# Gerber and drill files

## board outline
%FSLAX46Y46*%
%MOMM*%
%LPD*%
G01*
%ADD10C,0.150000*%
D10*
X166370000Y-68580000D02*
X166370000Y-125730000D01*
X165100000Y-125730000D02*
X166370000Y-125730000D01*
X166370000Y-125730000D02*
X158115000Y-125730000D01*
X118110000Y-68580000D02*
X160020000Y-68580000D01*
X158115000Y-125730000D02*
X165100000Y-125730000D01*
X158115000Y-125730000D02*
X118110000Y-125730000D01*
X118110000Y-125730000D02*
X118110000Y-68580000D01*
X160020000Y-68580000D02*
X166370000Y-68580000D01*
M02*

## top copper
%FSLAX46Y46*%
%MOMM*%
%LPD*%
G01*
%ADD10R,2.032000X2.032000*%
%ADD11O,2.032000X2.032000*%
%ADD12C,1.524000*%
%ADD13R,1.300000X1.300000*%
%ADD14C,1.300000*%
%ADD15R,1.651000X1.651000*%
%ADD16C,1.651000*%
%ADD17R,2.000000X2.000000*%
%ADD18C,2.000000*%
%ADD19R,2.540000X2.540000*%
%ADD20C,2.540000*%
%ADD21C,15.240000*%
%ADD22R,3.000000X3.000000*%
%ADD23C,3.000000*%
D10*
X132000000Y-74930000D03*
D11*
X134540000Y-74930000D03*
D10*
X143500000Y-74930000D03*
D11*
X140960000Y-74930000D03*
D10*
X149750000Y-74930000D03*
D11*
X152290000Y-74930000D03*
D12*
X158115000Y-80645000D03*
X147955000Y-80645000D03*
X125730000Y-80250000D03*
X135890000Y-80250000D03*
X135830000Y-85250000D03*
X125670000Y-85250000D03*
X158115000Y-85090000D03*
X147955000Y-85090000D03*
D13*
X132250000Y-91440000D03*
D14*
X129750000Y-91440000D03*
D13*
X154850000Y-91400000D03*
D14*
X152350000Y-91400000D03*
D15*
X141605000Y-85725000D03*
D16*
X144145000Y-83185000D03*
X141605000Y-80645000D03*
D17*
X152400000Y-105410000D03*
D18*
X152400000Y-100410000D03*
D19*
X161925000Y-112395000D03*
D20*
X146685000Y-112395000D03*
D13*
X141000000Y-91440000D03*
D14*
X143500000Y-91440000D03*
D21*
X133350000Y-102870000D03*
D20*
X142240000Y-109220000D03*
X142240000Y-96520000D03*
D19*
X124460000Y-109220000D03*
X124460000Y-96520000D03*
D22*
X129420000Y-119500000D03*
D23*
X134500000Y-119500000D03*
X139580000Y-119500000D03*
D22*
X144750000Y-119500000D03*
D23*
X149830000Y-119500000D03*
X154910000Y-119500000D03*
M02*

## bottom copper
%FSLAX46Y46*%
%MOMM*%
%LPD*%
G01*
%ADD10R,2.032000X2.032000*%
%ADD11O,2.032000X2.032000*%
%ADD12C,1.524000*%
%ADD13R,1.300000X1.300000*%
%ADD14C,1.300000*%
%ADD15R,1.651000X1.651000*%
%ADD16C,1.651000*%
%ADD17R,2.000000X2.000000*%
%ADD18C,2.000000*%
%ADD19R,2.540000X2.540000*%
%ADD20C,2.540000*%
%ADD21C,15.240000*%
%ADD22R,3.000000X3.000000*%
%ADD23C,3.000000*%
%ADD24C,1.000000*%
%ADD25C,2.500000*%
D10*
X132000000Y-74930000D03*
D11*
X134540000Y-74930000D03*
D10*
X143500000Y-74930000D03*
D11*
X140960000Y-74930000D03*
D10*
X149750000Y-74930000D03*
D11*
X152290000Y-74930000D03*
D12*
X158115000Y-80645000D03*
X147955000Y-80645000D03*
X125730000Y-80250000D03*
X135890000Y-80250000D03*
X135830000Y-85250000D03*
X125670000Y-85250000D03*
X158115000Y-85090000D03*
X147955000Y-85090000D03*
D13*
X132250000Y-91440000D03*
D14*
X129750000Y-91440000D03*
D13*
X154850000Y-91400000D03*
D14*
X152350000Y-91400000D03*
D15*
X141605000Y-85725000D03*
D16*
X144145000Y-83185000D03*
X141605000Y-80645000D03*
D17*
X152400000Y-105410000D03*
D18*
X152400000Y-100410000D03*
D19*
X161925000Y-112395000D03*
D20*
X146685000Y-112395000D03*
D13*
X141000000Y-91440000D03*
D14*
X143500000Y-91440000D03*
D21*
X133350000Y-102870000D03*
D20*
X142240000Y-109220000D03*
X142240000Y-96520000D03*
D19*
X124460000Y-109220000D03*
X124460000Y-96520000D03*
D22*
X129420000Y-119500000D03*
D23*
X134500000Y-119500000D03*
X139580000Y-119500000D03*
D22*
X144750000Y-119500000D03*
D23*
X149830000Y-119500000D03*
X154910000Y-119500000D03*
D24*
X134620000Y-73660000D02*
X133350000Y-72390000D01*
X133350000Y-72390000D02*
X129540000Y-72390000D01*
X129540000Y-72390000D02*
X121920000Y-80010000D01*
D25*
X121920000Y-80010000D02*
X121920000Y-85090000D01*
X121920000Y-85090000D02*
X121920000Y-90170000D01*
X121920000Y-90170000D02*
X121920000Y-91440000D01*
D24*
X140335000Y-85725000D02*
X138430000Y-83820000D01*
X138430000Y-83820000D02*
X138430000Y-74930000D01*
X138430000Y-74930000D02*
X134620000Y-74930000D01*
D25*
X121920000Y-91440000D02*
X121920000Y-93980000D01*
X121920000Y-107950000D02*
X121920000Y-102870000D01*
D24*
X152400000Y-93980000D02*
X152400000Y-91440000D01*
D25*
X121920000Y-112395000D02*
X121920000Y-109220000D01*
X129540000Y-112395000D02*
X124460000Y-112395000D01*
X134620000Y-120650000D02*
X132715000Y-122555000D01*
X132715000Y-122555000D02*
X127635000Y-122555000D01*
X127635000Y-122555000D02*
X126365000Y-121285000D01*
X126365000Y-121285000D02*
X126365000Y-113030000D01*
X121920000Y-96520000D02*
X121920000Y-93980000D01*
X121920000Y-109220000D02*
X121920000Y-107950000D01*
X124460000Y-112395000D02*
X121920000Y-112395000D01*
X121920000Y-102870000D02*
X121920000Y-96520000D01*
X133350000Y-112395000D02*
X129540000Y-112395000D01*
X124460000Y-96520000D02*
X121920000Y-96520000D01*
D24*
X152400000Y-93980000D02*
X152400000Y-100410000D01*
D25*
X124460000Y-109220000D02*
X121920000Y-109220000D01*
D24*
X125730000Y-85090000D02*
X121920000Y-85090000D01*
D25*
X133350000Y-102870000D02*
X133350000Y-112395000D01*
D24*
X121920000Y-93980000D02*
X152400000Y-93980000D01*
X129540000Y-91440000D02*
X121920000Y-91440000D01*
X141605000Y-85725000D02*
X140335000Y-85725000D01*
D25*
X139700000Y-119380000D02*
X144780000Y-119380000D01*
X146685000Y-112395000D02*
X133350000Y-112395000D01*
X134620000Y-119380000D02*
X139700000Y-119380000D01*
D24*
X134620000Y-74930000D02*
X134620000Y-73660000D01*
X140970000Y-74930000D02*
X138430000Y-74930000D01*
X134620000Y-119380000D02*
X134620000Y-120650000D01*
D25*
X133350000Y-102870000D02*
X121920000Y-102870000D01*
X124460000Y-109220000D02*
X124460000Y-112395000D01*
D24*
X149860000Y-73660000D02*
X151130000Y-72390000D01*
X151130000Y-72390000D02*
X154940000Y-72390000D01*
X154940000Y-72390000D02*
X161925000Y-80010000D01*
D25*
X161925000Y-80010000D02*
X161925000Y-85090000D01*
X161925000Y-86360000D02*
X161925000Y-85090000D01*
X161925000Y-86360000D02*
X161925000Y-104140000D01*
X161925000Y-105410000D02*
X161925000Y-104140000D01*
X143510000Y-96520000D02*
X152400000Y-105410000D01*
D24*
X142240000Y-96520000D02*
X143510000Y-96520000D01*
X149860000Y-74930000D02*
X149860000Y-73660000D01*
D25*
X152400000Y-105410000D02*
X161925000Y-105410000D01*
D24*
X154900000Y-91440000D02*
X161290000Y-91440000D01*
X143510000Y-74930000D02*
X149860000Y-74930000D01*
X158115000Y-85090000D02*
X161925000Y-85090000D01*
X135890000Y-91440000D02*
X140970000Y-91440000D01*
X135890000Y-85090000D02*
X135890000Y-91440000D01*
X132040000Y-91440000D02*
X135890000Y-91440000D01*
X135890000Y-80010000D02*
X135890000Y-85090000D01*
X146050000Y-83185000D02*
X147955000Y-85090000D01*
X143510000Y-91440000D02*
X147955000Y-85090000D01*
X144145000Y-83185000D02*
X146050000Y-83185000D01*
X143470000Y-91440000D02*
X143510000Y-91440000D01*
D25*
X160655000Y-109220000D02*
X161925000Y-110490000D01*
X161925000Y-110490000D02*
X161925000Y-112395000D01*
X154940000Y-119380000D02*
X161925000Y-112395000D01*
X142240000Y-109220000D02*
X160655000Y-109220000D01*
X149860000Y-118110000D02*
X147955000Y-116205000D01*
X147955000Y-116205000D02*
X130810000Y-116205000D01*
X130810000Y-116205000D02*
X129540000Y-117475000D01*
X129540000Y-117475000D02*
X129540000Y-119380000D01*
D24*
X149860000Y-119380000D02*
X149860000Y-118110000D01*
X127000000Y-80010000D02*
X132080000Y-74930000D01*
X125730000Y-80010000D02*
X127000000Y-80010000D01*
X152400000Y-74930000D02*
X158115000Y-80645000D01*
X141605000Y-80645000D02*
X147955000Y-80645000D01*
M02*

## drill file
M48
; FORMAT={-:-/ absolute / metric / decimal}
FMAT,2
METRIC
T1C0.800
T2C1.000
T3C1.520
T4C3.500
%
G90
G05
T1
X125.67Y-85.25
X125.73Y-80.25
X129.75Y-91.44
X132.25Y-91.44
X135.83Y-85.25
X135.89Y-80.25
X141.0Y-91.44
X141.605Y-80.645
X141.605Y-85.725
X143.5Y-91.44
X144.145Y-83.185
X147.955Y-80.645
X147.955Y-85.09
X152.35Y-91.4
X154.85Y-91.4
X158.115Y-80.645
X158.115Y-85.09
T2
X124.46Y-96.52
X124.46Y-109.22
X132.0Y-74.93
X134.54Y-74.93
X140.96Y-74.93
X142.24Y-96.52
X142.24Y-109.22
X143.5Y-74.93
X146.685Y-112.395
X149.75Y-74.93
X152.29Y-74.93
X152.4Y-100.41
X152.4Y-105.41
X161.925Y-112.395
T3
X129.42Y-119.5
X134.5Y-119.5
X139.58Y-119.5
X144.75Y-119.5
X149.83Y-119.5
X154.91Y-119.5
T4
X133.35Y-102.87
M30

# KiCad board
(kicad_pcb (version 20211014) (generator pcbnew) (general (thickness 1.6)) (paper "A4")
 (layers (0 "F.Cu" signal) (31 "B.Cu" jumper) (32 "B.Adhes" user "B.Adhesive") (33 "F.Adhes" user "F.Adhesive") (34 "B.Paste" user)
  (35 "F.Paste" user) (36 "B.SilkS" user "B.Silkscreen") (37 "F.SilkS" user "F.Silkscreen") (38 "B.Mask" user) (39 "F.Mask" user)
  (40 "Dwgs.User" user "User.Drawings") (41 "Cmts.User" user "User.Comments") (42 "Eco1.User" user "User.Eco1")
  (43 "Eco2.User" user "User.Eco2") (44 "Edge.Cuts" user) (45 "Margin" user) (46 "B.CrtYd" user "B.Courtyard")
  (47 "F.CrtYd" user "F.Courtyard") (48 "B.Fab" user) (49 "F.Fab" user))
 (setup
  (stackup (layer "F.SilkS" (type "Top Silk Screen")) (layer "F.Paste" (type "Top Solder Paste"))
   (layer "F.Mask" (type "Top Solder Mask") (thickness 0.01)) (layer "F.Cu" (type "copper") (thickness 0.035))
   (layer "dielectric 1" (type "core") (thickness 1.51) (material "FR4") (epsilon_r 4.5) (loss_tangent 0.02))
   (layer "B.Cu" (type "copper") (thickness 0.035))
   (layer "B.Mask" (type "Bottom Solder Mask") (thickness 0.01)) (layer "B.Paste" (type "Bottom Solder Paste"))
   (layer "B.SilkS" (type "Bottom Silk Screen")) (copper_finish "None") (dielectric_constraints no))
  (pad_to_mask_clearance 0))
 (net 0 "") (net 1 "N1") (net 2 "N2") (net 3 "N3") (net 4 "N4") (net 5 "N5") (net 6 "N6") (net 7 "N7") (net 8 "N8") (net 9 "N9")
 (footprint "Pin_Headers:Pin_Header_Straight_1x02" (layer "F.Cu") (at 132 74.93 90)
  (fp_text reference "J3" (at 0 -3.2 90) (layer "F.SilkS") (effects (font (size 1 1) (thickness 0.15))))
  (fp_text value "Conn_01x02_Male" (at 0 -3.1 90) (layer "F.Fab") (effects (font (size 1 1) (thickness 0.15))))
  (pad "1" thru_hole rect locked (at 0 0 90) (size 2.032 2.032) (drill 1) (layers *.Cu *.Mask) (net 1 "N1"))
  (pad "2" thru_hole oval locked (at 0 2.54 90) (size 2.032 2.032) (drill 1) (layers *.Cu *.Mask) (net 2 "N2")))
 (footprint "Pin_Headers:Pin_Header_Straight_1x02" (layer "F.Cu") (at 143.5 74.93 -90)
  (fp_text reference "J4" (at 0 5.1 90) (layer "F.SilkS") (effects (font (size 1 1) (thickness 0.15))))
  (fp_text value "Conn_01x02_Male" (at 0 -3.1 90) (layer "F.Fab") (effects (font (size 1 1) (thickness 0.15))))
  (pad "1" thru_hole rect locked (at 0 0 270) (size 2.032 2.032) (drill 1) (layers *.Cu *.Mask) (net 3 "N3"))
  (pad "2" thru_hole oval locked (at 0 2.54 270) (size 2.032 2.032) (drill 1) (layers *.Cu *.Mask) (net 2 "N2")))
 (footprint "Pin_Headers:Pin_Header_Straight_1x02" (layer "F.Cu") (at 149.75 74.93 90)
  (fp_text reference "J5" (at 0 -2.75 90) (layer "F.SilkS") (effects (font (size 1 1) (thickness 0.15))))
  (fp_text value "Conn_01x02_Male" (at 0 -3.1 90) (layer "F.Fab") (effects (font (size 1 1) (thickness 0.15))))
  (pad "1" thru_hole rect locked (at 0 0 90) (size 2.032 2.032) (drill 1) (layers *.Cu *.Mask) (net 3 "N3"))
  (pad "2" thru_hole oval locked (at 0 2.54 90) (size 2.032 2.032) (drill 1) (layers *.Cu *.Mask) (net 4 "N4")))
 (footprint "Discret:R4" (layer "F.Cu") (at 153.035 80.645 180)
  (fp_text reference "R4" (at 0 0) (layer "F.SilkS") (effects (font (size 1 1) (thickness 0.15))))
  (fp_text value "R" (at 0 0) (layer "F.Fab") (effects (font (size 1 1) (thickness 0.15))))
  (pad "1" thru_hole circle locked (at -5.08 0 180) (size 1.524 1.524) (drill 0.8) (layers *.Cu *.Mask) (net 4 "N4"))
  (pad "2" thru_hole circle locked (at 5.08 0 180) (size 1.524 1.524) (drill 0.8) (layers *.Cu *.Mask) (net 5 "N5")))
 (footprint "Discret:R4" (layer "F.Cu") (at 130.81 80.25)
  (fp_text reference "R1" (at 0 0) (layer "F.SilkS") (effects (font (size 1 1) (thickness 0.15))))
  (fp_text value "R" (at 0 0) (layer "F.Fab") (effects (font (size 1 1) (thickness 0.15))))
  (pad "1" thru_hole circle locked (at -5.08 0) (size 1.524 1.524) (drill 0.8) (layers *.Cu *.Mask) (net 1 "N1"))
  (pad "2" thru_hole circle locked (at 5.08 0) (size 1.524 1.524) (drill 0.8) (layers *.Cu *.Mask) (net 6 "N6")))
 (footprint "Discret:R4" (layer "F.Cu") (at 130.75 85.25 180)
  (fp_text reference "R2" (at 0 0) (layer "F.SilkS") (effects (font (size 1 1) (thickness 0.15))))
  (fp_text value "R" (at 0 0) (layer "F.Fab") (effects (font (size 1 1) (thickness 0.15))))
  (pad "1" thru_hole circle locked (at -5.08 0 180) (size 1.524 1.524) (drill 0.8) (layers *.Cu *.Mask) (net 6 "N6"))
  (pad "2" thru_hole circle locked (at 5.08 0 180) (size 1.524 1.524) (drill 0.8) (layers *.Cu *.Mask) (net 2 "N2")))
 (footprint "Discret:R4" (layer "F.Cu") (at 153.035 85.09 180)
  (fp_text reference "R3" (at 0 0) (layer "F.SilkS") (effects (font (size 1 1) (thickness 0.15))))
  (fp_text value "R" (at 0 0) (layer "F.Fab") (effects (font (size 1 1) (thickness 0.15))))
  (pad "1" thru_hole circle locked (at -5.08 0 180) (size 1.524 1.524) (drill 0.8) (layers *.Cu *.Mask) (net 3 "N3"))
  (pad "2" thru_hole circle locked (at 5.08 0 180) (size 1.524 1.524) (drill 0.8) (layers *.Cu *.Mask) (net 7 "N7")))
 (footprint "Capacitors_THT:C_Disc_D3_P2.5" (layer "F.Cu") (at 132.25 91.44 180)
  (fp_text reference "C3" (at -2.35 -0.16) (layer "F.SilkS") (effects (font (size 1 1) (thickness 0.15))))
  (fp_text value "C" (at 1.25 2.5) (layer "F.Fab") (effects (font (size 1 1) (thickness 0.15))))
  (pad "1" thru_hole rect locked (at 0 0 180) (size 1.3 1.3) (drill 0.8) (layers *.Cu *.Mask) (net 6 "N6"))
  (pad "2" thru_hole circle locked (at 2.5 0 180) (size 1.3 1.3) (drill 0.8) (layers *.Cu *.Mask) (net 2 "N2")))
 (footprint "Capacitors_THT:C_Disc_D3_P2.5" (layer "F.Cu") (at 154.85 91.4 180)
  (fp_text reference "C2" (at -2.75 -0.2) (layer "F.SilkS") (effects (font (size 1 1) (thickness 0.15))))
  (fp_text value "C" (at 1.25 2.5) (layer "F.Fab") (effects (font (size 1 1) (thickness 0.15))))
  (pad "1" thru_hole rect locked (at 0 0 180) (size 1.3 1.3) (drill 0.8) (layers *.Cu *.Mask) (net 3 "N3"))
  (pad "2" thru_hole circle locked (at 2.5 0 180) (size 1.3 1.3) (drill 0.8) (layers *.Cu *.Mask) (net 2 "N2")))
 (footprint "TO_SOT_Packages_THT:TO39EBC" (layer "F.Cu") (at 141.605 85.725 90)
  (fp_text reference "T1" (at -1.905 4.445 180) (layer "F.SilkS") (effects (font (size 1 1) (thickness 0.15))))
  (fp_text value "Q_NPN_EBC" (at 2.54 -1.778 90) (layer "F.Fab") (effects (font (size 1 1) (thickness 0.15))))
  (pad "1" thru_hole rect locked (at 0 0 90) (size 1.651 1.651) (drill 0.8) (layers *.Cu *.Mask) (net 2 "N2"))
  (pad "2" thru_hole circle locked (at 2.54 2.54 90) (size 1.651 1.651) (drill 0.8) (layers *.Cu *.Mask) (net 7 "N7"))
  (pad "3" thru_hole circle locked (at 5.08 0 90) (size 1.651 1.651) (drill 0.8) (layers *.Cu *.Mask) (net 5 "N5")))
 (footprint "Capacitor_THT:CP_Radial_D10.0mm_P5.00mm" (layer "F.Cu") (at 152.4 105.41 90)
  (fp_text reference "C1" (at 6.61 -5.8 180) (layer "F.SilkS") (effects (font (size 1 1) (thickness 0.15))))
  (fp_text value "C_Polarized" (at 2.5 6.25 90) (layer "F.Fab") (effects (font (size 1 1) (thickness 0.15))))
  (pad "1" thru_hole rect (at 0 0 90) (size 2 2) (drill 1) (layers *.Cu *.Mask) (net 3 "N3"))
  (pad "2" thru_hole circle (at 5 0 90) (size 2 2) (drill 1) (layers *.Cu *.Mask) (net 2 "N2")))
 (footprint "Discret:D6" (layer "F.Cu") (at 154.305 112.395)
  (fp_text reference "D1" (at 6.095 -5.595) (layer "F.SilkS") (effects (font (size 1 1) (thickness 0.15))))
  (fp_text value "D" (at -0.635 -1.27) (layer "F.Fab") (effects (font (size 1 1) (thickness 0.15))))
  (pad "1" thru_hole rect locked (at 7.62 0) (size 2.54 2.54) (drill 1) (layers *.Cu *.Mask) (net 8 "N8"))
  (pad "2" thru_hole circle locked (at -7.62 0) (size 2.54 2.54) (drill 1) (layers *.Cu *.Mask) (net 2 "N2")))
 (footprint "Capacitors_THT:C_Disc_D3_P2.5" (layer "F.Cu") (at 141 91.44)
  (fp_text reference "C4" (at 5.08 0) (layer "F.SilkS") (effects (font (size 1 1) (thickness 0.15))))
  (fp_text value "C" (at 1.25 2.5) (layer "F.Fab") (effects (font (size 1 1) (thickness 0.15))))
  (pad "1" thru_hole rect locked (at 0 0) (size 1.3 1.3) (drill 0.8) (layers *.Cu *.Mask) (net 6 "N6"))
  (pad "2" thru_hole circle locked (at 2.5 0) (size 1.3 1.3) (drill 0.8) (layers *.Cu *.Mask) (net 7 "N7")))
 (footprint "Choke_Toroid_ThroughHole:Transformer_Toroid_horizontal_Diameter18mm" (layer "F.Cu") (at 133.35 102.87 180)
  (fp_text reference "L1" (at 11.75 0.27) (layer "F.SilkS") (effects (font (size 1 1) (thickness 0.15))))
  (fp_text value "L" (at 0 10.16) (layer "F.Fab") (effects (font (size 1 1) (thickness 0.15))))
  (pad "" thru_hole circle locked (at 0 0 180) (size 15.24 15.24) (drill 3.5) (layers *.Cu *.SilkS *.Mask))
  (pad "1" thru_hole circle locked (at -8.89 -6.35 180) (size 2.54 2.54) (drill 1) (layers *.Cu *.SilkS *.Mask) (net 8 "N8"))
  (pad "2" thru_hole circle locked (at -8.89 6.35 180) (size 2.54 2.54) (drill 1) (layers *.Cu *.SilkS *.Mask) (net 3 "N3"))
  (pad "3" thru_hole rect locked (at 8.89 -6.35 180) (size 2.54 2.54) (drill 1) (layers *.Cu *.SilkS *.Mask))
  (pad "4" thru_hole rect locked (at 8.89 6.35 180) (size 2.54 2.54) (drill 1) (layers *.Cu *.SilkS *.Mask)))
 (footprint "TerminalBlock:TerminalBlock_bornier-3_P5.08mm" (layer "F.Cu") (at 129.42 119.5)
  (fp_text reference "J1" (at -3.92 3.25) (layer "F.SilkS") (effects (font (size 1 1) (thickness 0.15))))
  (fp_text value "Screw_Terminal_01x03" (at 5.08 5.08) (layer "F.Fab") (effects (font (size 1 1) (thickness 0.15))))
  (pad "1" thru_hole rect (at 0 0) (size 3 3) (drill 1.52) (layers *.Cu *.Mask) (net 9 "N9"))
  (pad "2" thru_hole circle (at 5.08 0) (size 3 3) (drill 1.52) (layers *.Cu *.Mask) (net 2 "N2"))
  (pad "3" thru_hole circle (at 10.16 0) (size 3 3) (drill 1.52) (layers *.Cu *.Mask) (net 2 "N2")))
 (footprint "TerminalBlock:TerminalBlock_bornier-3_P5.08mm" (layer "F.Cu") (at 144.75 119.5)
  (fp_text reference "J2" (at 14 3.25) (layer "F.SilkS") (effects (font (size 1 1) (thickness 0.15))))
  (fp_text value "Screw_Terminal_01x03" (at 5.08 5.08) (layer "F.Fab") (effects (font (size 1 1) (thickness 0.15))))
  (pad "1" thru_hole rect (at 0 0) (size 3 3) (drill 1.52) (layers *.Cu *.Mask) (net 2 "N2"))
  (pad "2" thru_hole circle (at 5.08 0) (size 3 3) (drill 1.52) (layers *.Cu *.Mask) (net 9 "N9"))
  (pad "3" thru_hole circle (at 10.16 0) (size 3 3) (drill 1.52) (layers *.Cu *.Mask) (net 8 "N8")))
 (gr_line (start 166.37 68.58) (end 166.37 125.73) (layer "Edge.Cuts") (width 0.15))
 (gr_line (start 165.1 125.73) (end 166.37 125.73) (layer "Edge.Cuts") (width 0.15))
 (gr_line (start 166.37 125.73) (end 158.115 125.73) (layer "Edge.Cuts") (width 0.15))
 (gr_line (start 118.11 68.58) (end 160.02 68.58) (layer "Edge.Cuts") (width 0.15))
 (gr_line (start 158.115 125.73) (end 165.1 125.73) (layer "Edge.Cuts") (width 0.15))
 (gr_line (start 158.115 125.73) (end 118.11 125.73) (layer "Edge.Cuts") (width 0.15))
 (gr_line (start 118.11 125.73) (end 118.11 68.58) (layer "Edge.Cuts") (width 0.15))
 (gr_line (start 160.02 68.58) (end 166.37 68.58) (layer "Edge.Cuts") (width 0.15))
 (segment (start 134.62 73.66) (end 133.35 72.39) (width 1) (layer "B.Cu") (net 2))
 (segment (start 133.35 72.39) (end 129.54 72.39) (width 1) (layer "B.Cu") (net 2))
 (segment (start 129.54 72.39) (end 121.92 80.01) (width 1) (layer "B.Cu") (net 2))
 (segment (start 121.92 80.01) (end 121.92 85.09) (width 2.5) (layer "B.Cu") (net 2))
 (segment (start 121.92 85.09) (end 121.92 90.17) (width 2.5) (layer "B.Cu") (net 2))
 (segment (start 121.92 90.17) (end 121.92 91.44) (width 2.5) (layer "B.Cu") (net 2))
 (segment (start 140.335 85.725) (end 138.43 83.82) (width 1) (layer "B.Cu") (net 2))
 (segment (start 138.43 83.82) (end 138.43 74.93) (width 1) (layer "B.Cu") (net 2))
 (segment (start 138.43 74.93) (end 134.62 74.93) (width 1) (layer "B.Cu") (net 2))
 (segment (start 121.92 91.44) (end 121.92 93.98) (width 2.5) (layer "B.Cu") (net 2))
 (segment (start 121.92 107.95) (end 121.92 102.87) (width 2.5) (layer "B.Cu") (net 2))
 (segment (start 152.4 93.98) (end 152.4 91.44) (width 1) (layer "B.Cu") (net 2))
 (segment (start 121.92 112.395) (end 121.92 109.22) (width 2.5) (layer "B.Cu") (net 2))
 (segment (start 129.54 112.395) (end 124.46 112.395) (width 2.5) (layer "B.Cu") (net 2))
 (segment (start 134.62 120.65) (end 132.715 122.555) (width 2.5) (layer "B.Cu") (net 2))
 (segment (start 132.715 122.555) (end 127.635 122.555) (width 2.5) (layer "B.Cu") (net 2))
 (segment (start 127.635 122.555) (end 126.365 121.285) (width 2.5) (layer "B.Cu") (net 2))
 (segment (start 126.365 121.285) (end 126.365 113.03) (width 2.5) (layer "B.Cu") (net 2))
 (segment (start 121.92 96.52) (end 121.92 93.98) (width 2.5) (layer "B.Cu") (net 2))
 (segment (start 121.92 109.22) (end 121.92 107.95) (width 2.5) (layer "B.Cu") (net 2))
 (segment (start 124.46 112.395) (end 121.92 112.395) (width 2.5) (layer "B.Cu") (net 2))
 (segment (start 121.92 102.87) (end 121.92 96.52) (width 2.5) (layer "B.Cu") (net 2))
 (segment (start 133.35 112.395) (end 129.54 112.395) (width 2.5) (layer "B.Cu") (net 2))
 (segment (start 124.46 96.52) (end 121.92 96.52) (width 2.5) (layer "B.Cu") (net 2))
 (segment (start 152.4 93.98) (end 152.4 100.41) (width 1) (layer "B.Cu") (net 2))
 (segment (start 124.46 109.22) (end 121.92 109.22) (width 2.5) (layer "B.Cu") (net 2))
 (segment (start 125.73 85.09) (end 121.92 85.09) (width 1) (layer "B.Cu") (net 2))
 (segment (start 133.35 102.87) (end 133.35 112.395) (width 2.5) (layer "B.Cu") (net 2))
 (segment (start 121.92 93.98) (end 152.4 93.98) (width 1) (layer "B.Cu") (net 2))
 (segment (start 129.54 91.44) (end 121.92 91.44) (width 1) (layer "B.Cu") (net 2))
 (segment (start 141.605 85.725) (end 140.335 85.725) (width 1) (layer "B.Cu") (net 2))
 (segment (start 139.7 119.38) (end 144.78 119.38) (width 2.5) (layer "B.Cu") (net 2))
 (segment (start 146.685 112.395) (end 133.35 112.395) (width 2.5) (layer "B.Cu") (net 2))
 (segment (start 134.62 119.38) (end 139.7 119.38) (width 2.5) (layer "B.Cu") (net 2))
 (segment (start 134.62 74.93) (end 134.62 73.66) (width 1) (layer "B.Cu") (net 2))
 (segment (start 140.97 74.93) (end 138.43 74.93) (width 1) (layer "B.Cu") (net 2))
 (segment (start 134.62 119.38) (end 134.62 120.65) (width 1) (layer "B.Cu") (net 2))
 (segment (start 133.35 102.87) (end 121.92 102.87) (width 2.5) (layer "B.Cu") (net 2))
 (segment (start 124.46 109.22) (end 124.46 112.395) (width 2.5) (layer "B.Cu") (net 2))
 (segment (start 149.86 73.66) (end 151.13 72.39) (width 1) (layer "B.Cu") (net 3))
 (segment (start 151.13 72.39) (end 154.94 72.39) (width 1) (layer "B.Cu") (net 3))
 (segment (start 154.94 72.39) (end 161.925 80.01) (width 1) (layer "B.Cu") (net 3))
 (segment (start 161.925 80.01) (end 161.925 85.09) (width 2.5) (layer "B.Cu") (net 3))
 (segment (start 161.925 86.36) (end 161.925 85.09) (width 2.5) (layer "B.Cu") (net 3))
 (segment (start 161.925 86.36) (end 161.925 104.14) (width 2.5) (layer "B.Cu") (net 3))
 (segment (start 161.925 105.41) (end 161.925 104.14) (width 2.5) (layer "B.Cu") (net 3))
 (segment (start 143.51 96.52) (end 152.4 105.41) (width 2.5) (layer "B.Cu") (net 3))
 (segment (start 142.24 96.52) (end 143.51 96.52) (width 1) (layer "B.Cu") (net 3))
 (segment (start 149.86 74.93) (end 149.86 73.66) (width 1) (layer "B.Cu") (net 3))
 (segment (start 152.4 105.41) (end 161.925 105.41) (width 2.5) (layer "B.Cu") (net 3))
 (segment (start 154.9 91.44) (end 161.29 91.44) (width 1) (layer "B.Cu") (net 3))
 (segment (start 143.51 74.93) (end 149.86 74.93) (width 1) (layer "B.Cu") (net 3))
 (segment (start 158.115 85.09) (end 161.925 85.09) (width 1) (layer "B.Cu") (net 3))
 (segment (start 135.89 91.44) (end 140.97 91.44) (width 1) (layer "B.Cu") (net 6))
 (segment (start 135.89 85.09) (end 135.89 91.44) (width 1) (layer "B.Cu") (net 6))
 (segment (start 132.04 91.44) (end 135.89 91.44) (width 1) (layer "B.Cu") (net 6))
 (segment (start 135.89 80.01) (end 135.89 85.09) (width 1) (layer "B.Cu") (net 6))
 (segment (start 146.05 83.185) (end 147.955 85.09) (width 1) (layer "B.Cu") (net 7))
 (segment (start 143.51 91.44) (end 147.955 85.09) (width 1) (layer "B.Cu") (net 7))
 (segment (start 144.145 83.185) (end 146.05 83.185) (width 1) (layer "B.Cu") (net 7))
 (segment (start 143.47 91.44) (end 143.51 91.44) (width 1) (layer "B.Cu") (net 7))
 (segment (start 160.655 109.22) (end 161.925 110.49) (width 2.5) (layer "B.Cu") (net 8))
 (segment (start 161.925 110.49) (end 161.925 112.395) (width 2.5) (layer "B.Cu") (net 8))
 (segment (start 154.94 119.38) (end 161.925 112.395) (width 2.5) (layer "B.Cu") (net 8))
 (segment (start 142.24 109.22) (end 160.655 109.22) (width 2.5) (layer "B.Cu") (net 8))
 (segment (start 149.86 118.11) (end 147.955 116.205) (width 2.5) (layer "B.Cu") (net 9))
 (segment (start 147.955 116.205) (end 130.81 116.205) (width 2.5) (layer "B.Cu") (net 9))
 (segment (start 130.81 116.205) (end 129.54 117.475) (width 2.5) (layer "B.Cu") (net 9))
 (segment (start 129.54 117.475) (end 129.54 119.38) (width 2.5) (layer "B.Cu") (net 9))
 (segment (start 149.86 119.38) (end 149.86 118.11) (width 1) (layer "B.Cu") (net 9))
 (segment (start 127 80.01) (end 132.08 74.93) (width 1) (layer "B.Cu") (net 1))
 (segment (start 125.73 80.01) (end 127 80.01) (width 1) (layer "B.Cu") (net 1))
 (segment (start 152.4 74.93) (end 158.115 80.645) (width 1) (layer "B.Cu") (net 4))
 (segment (start 141.605 80.645) (end 147.955 80.645) (width 1) (layer "B.Cu") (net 5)))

